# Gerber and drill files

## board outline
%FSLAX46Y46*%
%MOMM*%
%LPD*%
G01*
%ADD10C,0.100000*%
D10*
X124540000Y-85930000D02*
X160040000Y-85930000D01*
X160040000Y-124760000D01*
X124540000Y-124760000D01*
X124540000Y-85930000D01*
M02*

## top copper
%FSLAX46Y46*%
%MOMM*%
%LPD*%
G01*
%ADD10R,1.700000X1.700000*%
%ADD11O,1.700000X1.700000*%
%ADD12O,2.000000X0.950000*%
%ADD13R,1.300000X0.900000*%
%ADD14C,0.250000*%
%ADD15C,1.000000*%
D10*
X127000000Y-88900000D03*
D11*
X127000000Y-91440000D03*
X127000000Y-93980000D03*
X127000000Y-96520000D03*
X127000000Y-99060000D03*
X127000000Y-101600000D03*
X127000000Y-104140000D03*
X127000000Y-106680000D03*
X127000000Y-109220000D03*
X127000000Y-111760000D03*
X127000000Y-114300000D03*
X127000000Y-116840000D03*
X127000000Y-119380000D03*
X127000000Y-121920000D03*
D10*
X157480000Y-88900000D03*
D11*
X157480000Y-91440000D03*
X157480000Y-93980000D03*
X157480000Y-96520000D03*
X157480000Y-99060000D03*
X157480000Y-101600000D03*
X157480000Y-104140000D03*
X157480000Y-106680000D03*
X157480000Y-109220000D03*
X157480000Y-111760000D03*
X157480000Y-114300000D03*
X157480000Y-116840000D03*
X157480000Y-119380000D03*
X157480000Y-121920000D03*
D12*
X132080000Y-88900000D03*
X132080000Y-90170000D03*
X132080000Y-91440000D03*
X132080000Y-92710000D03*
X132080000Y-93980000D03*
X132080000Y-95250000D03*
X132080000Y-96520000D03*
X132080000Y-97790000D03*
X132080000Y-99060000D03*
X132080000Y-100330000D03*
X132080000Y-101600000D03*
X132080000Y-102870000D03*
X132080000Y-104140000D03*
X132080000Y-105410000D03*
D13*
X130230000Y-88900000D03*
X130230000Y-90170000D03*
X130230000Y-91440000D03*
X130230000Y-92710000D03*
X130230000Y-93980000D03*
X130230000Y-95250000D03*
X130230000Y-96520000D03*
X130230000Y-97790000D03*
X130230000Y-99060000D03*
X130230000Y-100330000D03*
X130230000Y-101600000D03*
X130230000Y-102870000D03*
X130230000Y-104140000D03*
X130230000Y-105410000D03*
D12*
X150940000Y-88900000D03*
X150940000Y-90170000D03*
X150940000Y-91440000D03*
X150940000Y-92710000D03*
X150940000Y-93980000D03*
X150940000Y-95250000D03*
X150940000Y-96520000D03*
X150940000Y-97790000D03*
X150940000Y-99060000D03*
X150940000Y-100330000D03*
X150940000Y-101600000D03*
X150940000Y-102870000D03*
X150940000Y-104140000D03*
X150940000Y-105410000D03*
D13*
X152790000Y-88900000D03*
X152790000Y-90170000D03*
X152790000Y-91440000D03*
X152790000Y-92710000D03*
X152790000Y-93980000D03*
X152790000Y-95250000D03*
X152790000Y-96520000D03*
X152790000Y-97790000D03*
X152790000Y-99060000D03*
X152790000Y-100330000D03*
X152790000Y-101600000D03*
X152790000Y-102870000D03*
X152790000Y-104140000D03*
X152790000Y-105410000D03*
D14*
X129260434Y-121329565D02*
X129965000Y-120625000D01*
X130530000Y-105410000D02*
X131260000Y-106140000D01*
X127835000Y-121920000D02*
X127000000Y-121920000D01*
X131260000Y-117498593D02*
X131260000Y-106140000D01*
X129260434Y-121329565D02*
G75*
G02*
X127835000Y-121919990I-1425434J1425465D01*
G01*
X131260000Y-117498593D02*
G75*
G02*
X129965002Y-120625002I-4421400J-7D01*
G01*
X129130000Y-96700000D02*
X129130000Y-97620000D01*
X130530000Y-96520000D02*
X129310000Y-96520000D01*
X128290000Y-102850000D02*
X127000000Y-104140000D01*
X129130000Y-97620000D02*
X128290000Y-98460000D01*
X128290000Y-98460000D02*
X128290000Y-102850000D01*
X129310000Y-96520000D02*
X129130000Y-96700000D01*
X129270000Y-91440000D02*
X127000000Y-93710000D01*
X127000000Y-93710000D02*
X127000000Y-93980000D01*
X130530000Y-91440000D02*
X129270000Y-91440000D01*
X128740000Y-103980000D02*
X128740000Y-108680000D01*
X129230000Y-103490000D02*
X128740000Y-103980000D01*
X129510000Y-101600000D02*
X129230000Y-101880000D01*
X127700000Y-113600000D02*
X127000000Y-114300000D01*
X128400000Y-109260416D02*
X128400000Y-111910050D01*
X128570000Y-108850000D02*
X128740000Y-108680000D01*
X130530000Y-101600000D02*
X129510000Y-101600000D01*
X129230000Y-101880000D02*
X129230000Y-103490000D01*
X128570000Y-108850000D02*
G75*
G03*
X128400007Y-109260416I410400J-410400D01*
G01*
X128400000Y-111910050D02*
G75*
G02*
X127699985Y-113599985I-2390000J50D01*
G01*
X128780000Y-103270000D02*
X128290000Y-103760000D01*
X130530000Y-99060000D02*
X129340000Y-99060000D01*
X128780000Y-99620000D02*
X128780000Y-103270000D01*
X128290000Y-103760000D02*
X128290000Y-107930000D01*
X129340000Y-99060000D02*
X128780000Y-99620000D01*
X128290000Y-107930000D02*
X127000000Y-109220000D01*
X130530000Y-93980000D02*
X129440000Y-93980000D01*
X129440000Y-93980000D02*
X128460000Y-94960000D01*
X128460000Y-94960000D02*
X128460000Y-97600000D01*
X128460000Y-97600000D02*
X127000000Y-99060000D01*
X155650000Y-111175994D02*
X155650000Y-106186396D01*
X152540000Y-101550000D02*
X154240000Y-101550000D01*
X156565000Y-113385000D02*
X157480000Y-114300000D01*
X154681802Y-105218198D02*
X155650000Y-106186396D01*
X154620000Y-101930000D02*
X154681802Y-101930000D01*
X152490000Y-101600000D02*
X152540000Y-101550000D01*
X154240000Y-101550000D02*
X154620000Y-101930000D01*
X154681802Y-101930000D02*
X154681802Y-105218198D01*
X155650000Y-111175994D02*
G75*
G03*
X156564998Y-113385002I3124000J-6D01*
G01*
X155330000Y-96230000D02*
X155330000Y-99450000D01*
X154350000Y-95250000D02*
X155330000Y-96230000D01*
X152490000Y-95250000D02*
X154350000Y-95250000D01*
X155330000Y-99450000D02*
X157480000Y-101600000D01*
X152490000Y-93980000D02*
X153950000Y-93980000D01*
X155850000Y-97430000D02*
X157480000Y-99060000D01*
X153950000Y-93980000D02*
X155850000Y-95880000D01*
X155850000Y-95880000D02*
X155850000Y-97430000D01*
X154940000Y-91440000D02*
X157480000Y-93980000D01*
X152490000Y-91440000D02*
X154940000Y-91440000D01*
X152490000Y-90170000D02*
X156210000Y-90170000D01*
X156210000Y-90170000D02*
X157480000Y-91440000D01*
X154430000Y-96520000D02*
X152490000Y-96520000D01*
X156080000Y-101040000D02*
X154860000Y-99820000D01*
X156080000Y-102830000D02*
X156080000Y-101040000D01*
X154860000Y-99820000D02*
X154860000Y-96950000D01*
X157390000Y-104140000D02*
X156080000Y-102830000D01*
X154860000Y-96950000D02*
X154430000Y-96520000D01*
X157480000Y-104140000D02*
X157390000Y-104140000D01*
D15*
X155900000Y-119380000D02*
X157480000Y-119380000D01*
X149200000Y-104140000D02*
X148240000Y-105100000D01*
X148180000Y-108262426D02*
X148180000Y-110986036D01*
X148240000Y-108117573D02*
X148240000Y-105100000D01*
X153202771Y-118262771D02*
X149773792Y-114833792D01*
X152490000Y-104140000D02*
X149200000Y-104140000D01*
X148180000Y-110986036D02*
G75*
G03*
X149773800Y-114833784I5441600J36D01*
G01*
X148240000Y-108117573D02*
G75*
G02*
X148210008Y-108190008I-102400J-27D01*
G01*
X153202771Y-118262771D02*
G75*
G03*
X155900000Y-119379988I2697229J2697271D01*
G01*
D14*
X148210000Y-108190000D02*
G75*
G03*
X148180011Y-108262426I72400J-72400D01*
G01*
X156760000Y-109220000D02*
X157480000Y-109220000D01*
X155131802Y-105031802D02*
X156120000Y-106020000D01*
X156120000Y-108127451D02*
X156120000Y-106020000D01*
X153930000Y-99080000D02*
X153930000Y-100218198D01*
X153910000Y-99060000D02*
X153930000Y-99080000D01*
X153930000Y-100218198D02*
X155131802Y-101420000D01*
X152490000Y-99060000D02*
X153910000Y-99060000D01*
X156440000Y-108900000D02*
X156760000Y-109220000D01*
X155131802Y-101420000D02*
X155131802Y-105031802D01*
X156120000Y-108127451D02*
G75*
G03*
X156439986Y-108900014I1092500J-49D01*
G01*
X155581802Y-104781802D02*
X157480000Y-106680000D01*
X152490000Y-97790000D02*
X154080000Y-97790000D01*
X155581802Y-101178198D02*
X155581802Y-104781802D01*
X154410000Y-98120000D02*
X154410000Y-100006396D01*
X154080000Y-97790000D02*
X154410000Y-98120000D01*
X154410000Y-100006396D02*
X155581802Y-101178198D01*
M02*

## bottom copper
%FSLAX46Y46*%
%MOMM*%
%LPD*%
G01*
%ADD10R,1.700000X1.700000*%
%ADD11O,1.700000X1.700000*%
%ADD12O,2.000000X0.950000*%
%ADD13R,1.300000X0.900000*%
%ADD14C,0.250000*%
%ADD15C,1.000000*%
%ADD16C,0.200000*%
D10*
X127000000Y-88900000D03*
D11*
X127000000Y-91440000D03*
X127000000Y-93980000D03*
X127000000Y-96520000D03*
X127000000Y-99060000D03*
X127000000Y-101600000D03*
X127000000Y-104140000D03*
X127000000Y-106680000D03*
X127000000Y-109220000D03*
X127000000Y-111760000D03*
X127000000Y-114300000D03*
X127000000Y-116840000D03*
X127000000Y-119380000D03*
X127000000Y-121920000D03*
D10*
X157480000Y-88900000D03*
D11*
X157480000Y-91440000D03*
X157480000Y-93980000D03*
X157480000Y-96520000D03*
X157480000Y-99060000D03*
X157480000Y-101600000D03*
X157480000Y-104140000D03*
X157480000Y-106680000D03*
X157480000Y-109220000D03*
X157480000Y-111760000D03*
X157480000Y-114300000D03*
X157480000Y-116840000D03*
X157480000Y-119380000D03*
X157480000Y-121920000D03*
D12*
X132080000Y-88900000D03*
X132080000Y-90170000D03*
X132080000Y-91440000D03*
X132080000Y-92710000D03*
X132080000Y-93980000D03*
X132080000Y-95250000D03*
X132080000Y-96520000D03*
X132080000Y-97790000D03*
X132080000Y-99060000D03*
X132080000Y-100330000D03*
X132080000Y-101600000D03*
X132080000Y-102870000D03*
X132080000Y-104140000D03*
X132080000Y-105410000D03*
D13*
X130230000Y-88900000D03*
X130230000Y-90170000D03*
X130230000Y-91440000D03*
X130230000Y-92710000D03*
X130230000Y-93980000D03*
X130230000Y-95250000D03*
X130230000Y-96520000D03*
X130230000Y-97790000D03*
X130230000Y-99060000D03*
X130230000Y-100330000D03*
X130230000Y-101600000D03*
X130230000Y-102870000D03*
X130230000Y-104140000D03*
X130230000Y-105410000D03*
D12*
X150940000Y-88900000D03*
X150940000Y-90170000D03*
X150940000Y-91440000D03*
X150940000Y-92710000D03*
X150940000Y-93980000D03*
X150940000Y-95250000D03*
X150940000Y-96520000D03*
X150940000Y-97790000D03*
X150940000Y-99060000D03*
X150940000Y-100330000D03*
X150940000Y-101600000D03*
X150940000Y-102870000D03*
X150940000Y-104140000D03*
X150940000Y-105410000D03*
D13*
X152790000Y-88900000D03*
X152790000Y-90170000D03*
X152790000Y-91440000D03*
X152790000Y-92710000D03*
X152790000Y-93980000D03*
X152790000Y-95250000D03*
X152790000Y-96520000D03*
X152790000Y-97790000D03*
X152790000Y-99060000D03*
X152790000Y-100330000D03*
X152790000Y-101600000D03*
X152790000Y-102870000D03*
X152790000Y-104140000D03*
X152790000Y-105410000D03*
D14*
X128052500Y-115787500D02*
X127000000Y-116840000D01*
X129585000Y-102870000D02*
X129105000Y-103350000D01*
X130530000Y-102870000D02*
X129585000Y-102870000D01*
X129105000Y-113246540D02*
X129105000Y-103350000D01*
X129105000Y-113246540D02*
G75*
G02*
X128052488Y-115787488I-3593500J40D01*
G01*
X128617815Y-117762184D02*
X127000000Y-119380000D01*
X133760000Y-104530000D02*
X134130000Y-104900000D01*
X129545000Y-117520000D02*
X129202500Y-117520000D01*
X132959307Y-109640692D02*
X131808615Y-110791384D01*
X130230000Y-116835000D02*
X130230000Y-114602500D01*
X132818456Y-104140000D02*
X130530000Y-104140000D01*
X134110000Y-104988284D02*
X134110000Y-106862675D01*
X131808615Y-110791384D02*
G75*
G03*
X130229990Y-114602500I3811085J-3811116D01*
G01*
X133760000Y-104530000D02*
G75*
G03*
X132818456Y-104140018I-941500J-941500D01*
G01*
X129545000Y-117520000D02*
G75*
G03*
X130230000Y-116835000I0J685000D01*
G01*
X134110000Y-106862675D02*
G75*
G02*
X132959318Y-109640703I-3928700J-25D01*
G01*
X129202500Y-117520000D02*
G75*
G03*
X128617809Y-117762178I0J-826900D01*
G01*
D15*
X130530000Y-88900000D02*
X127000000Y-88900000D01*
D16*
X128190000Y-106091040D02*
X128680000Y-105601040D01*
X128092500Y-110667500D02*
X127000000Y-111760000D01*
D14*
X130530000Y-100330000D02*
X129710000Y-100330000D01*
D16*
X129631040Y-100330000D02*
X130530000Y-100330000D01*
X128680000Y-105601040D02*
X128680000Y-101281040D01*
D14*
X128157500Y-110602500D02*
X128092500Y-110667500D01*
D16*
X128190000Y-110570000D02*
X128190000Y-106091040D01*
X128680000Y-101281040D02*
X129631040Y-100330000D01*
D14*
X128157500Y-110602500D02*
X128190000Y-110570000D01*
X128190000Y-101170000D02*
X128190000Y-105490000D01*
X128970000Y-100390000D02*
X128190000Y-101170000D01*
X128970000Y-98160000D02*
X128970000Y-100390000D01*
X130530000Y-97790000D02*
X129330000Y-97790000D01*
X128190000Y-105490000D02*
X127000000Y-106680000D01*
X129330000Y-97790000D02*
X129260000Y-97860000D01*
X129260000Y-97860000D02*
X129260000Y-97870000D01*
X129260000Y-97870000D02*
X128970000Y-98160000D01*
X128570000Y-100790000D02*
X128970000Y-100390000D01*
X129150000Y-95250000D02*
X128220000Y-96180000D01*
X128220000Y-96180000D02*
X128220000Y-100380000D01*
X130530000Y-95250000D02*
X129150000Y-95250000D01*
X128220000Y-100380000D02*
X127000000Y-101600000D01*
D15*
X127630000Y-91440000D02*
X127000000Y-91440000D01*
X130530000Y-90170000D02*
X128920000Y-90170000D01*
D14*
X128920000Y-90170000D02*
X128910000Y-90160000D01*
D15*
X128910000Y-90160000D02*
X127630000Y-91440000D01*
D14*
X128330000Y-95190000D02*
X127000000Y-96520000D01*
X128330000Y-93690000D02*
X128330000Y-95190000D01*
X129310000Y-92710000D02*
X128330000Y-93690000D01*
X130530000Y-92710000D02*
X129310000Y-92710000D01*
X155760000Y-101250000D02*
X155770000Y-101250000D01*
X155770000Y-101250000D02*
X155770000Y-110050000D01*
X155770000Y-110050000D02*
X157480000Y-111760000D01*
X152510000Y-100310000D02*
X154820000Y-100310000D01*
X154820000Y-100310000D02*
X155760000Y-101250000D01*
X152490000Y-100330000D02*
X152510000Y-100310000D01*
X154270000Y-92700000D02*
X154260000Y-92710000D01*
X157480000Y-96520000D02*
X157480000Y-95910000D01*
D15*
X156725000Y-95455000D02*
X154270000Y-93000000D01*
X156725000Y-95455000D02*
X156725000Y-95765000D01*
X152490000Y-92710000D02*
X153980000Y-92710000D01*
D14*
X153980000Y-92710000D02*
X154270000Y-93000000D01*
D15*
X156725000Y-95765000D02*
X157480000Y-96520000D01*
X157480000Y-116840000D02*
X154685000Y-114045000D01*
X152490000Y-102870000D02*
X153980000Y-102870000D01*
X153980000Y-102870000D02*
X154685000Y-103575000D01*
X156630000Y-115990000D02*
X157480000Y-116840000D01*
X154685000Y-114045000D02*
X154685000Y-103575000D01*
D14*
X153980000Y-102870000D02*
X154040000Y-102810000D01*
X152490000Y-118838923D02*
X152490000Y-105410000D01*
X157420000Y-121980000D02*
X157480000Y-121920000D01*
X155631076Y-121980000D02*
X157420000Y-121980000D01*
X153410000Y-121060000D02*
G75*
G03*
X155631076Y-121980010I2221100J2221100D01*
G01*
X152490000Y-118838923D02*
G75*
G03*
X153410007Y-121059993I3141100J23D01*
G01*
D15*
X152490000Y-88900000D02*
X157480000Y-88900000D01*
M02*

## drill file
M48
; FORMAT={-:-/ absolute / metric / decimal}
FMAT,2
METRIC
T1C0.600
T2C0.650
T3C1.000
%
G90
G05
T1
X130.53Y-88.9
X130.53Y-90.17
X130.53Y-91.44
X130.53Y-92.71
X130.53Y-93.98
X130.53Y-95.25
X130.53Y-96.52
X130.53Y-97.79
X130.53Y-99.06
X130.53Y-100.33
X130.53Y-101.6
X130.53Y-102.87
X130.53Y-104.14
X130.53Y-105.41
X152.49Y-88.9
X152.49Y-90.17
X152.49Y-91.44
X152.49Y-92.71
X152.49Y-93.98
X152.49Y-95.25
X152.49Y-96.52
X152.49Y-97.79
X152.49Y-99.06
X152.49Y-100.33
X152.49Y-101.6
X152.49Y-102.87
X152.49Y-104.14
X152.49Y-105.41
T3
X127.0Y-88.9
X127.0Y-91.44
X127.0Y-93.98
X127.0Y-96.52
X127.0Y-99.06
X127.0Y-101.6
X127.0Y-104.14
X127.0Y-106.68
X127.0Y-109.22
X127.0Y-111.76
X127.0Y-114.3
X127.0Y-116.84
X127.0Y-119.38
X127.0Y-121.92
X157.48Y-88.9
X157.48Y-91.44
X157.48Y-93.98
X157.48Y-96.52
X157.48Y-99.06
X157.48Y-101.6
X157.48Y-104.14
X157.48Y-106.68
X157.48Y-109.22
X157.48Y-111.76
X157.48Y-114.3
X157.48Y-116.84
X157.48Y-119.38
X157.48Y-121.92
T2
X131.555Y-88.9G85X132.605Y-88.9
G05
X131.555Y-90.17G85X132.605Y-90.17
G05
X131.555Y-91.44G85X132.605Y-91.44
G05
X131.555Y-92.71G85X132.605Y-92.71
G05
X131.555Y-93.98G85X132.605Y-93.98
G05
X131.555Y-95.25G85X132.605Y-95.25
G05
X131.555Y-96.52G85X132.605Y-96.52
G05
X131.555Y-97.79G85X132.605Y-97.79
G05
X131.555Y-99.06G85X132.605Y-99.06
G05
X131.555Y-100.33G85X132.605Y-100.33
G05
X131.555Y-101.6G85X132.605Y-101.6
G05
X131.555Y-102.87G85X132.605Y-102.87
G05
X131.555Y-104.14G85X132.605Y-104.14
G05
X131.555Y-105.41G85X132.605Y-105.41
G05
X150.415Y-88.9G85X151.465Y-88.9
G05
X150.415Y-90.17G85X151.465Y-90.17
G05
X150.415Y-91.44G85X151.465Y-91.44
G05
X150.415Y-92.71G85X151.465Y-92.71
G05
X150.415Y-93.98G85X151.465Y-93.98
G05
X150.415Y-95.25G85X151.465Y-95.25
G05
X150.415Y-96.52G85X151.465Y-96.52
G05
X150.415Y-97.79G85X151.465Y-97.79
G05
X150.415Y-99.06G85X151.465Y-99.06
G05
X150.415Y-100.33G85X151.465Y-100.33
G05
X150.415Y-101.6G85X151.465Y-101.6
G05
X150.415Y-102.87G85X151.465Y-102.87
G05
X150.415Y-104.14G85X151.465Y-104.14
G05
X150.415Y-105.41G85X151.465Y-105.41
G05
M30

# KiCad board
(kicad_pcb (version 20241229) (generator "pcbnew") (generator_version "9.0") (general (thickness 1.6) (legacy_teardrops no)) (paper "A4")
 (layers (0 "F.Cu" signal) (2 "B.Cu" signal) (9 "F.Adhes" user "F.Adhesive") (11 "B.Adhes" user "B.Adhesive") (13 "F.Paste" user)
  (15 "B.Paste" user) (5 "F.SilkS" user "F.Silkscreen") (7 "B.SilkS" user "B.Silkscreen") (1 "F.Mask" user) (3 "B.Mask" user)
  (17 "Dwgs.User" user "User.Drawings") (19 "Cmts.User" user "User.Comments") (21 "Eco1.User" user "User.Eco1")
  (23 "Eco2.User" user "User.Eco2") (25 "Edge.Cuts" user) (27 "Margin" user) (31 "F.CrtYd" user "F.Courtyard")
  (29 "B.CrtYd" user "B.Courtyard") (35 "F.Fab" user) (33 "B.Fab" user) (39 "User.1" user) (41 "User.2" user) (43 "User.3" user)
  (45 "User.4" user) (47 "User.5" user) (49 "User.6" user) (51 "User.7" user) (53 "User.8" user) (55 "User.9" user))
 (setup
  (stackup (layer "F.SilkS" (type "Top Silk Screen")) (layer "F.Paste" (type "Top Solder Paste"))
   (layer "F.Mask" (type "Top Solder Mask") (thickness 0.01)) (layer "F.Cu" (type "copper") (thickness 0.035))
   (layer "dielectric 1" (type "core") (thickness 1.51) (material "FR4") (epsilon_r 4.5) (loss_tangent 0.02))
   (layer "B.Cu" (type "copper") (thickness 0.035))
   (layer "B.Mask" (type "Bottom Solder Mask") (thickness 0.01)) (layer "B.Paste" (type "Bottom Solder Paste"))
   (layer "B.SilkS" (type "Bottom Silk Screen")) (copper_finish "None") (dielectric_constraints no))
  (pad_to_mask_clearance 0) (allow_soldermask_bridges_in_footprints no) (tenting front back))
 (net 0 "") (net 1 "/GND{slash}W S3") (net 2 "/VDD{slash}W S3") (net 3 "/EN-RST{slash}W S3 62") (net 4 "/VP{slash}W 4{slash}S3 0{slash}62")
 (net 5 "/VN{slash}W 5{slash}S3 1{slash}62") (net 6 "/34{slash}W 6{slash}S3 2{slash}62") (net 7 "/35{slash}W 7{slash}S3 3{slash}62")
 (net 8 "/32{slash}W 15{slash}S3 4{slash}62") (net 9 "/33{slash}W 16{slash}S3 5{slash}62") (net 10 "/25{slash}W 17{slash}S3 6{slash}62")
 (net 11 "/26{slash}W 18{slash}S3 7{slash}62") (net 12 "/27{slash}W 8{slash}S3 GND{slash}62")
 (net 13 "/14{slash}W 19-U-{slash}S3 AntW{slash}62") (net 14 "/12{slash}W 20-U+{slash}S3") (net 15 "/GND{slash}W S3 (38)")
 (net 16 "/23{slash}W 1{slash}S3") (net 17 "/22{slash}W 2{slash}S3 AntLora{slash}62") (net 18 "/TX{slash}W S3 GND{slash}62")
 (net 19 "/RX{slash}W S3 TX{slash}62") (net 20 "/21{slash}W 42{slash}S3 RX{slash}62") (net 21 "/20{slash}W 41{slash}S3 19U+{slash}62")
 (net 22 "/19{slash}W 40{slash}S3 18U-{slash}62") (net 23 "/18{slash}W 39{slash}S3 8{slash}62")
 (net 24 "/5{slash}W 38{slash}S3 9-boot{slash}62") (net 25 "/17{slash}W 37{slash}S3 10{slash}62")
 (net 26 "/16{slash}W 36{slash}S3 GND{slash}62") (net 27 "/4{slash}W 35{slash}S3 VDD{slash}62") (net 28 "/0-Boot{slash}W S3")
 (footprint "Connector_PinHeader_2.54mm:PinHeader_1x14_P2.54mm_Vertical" (layer "F.Cu") (at 127 88.9)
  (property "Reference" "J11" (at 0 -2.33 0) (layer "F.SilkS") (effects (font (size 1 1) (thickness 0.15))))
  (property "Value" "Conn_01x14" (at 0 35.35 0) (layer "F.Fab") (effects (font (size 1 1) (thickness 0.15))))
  (pad "1" thru_hole rect (at 0 0) (size 1.7 1.7) (drill 1) (layers "*.Cu" "*.Mask") (remove_unused_layers no) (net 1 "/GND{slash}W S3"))
  (pad "2" thru_hole oval (at 0 2.54) (size 1.7 1.7) (drill 1) (layers "*.Cu" "*.Mask") (remove_unused_layers no) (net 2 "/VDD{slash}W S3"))
  (pad "3" thru_hole oval (at 0 5.08) (size 1.7 1.7) (drill 1) (layers "*.Cu" "*.Mask") (remove_unused_layers no)
   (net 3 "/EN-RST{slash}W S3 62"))
  (pad "4" thru_hole oval (at 0 7.62) (size 1.7 1.7) (drill 1) (layers "*.Cu" "*.Mask") (remove_unused_layers no)
   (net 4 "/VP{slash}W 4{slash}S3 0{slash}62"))
  (pad "5" thru_hole oval (at 0 10.16) (size 1.7 1.7) (drill 1) (layers "*.Cu" "*.Mask") (remove_unused_layers no)
   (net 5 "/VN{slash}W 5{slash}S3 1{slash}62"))
  (pad "6" thru_hole oval (at 0 12.7) (size 1.7 1.7) (drill 1) (layers "*.Cu" "*.Mask") (remove_unused_layers no)
   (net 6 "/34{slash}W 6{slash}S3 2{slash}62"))
  (pad "7" thru_hole oval (at 0 15.24) (size 1.7 1.7) (drill 1) (layers "*.Cu" "*.Mask") (remove_unused_layers no)
   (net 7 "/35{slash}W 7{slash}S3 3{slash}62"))
  (pad "8" thru_hole oval (at 0 17.78) (size 1.7 1.7) (drill 1) (layers "*.Cu" "*.Mask") (remove_unused_layers no)
   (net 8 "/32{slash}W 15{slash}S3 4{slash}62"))
  (pad "9" thru_hole oval (at 0 20.32) (size 1.7 1.7) (drill 1) (layers "*.Cu" "*.Mask") (remove_unused_layers no)
   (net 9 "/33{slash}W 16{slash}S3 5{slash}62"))
  (pad "10" thru_hole oval (at 0 22.86) (size 1.7 1.7) (drill 1) (layers "*.Cu" "*.Mask") (remove_unused_layers no)
   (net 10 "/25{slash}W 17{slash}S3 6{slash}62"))
  (pad "11" thru_hole oval (at 0 25.4) (size 1.7 1.7) (drill 1) (layers "*.Cu" "*.Mask") (remove_unused_layers no)
   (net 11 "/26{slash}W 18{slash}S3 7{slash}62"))
  (pad "12" thru_hole oval (at 0 27.94) (size 1.7 1.7) (drill 1) (layers "*.Cu" "*.Mask") (remove_unused_layers no)
   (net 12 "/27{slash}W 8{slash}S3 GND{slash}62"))
  (pad "13" thru_hole oval (at 0 30.48) (size 1.7 1.7) (drill 1) (layers "*.Cu" "*.Mask") (remove_unused_layers no)
   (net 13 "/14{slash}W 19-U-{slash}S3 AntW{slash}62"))
  (pad "14" thru_hole oval (at 0 33.02) (size 1.7 1.7) (drill 1) (layers "*.Cu" "*.Mask") (remove_unused_layers no)
   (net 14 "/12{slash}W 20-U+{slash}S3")))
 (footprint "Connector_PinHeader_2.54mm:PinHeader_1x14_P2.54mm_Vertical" (layer "F.Cu") (at 157.48 88.9)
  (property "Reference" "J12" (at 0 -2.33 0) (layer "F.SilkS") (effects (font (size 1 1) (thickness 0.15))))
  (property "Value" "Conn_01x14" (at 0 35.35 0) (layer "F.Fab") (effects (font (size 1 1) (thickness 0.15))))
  (pad "1" thru_hole rect (at 0 0) (size 1.7 1.7) (drill 1) (layers "*.Cu" "*.Mask") (remove_unused_layers no)
   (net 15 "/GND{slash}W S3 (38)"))
  (pad "2" thru_hole oval (at 0 2.54) (size 1.7 1.7) (drill 1) (layers "*.Cu" "*.Mask") (remove_unused_layers no)
   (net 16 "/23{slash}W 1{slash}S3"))
  (pad "3" thru_hole oval (at 0 5.08) (size 1.7 1.7) (drill 1) (layers "*.Cu" "*.Mask") (remove_unused_layers no)
   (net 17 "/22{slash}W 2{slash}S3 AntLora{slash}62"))
  (pad "4" thru_hole oval (at 0 7.62) (size 1.7 1.7) (drill 1) (layers "*.Cu" "*.Mask") (remove_unused_layers no)
   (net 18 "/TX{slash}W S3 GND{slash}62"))
  (pad "5" thru_hole oval (at 0 10.16) (size 1.7 1.7) (drill 1) (layers "*.Cu" "*.Mask") (remove_unused_layers no)
   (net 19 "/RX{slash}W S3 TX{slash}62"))
  (pad "6" thru_hole oval (at 0 12.7) (size 1.7 1.7) (drill 1) (layers "*.Cu" "*.Mask") (remove_unused_layers no)
   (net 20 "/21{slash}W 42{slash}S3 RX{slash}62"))
  (pad "7" thru_hole oval (at 0 15.24) (size 1.7 1.7) (drill 1) (layers "*.Cu" "*.Mask") (remove_unused_layers no)
   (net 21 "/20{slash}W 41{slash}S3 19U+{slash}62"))
  (pad "8" thru_hole oval (at 0 17.78) (size 1.7 1.7) (drill 1) (layers "*.Cu" "*.Mask") (remove_unused_layers no)
   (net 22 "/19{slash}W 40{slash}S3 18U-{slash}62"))
  (pad "9" thru_hole oval (at 0 20.32) (size 1.7 1.7) (drill 1) (layers "*.Cu" "*.Mask") (remove_unused_layers no)
   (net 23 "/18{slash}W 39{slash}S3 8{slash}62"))
  (pad "10" thru_hole oval (at 0 22.86) (size 1.7 1.7) (drill 1) (layers "*.Cu" "*.Mask") (remove_unused_layers no)
   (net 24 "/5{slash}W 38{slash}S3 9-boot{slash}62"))
  (pad "11" thru_hole oval (at 0 25.4) (size 1.7 1.7) (drill 1) (layers "*.Cu" "*.Mask") (remove_unused_layers no)
   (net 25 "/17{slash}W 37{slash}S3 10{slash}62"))
  (pad "12" thru_hole oval (at 0 27.94) (size 1.7 1.7) (drill 1) (layers "*.Cu" "*.Mask") (remove_unused_layers no)
   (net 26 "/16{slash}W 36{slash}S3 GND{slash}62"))
  (pad "13" thru_hole oval (at 0 30.48) (size 1.7 1.7) (drill 1) (layers "*.Cu" "*.Mask") (remove_unused_layers no)
   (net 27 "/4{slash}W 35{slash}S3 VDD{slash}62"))
  (pad "14" thru_hole oval (at 0 33.02) (size 1.7 1.7) (drill 1) (layers "*.Cu" "*.Mask") (remove_unused_layers no)
   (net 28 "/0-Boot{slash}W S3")))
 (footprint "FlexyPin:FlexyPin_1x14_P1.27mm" (layer "F.Cu") (at 130.53 88.9)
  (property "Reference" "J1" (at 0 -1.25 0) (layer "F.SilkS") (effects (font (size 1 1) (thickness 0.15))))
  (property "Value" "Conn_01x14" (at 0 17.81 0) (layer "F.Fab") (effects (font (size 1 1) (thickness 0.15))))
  (pad "" thru_hole oval (at 1.55 0) (size 2 0.95) (drill oval 1.7 0.65) (layers "*.Cu" "*.Mask") (remove_unused_layers no))
  (pad "" thru_hole oval (at 1.55 1.27) (size 2 0.95) (drill oval 1.7 0.65) (layers "*.Cu" "*.Mask") (remove_unused_layers no))
  (pad "" thru_hole oval (at 1.55 2.54) (size 2 0.95) (drill oval 1.7 0.65) (layers "*.Cu" "*.Mask") (remove_unused_layers no))
  (pad "" thru_hole oval (at 1.55 3.81) (size 2 0.95) (drill oval 1.7 0.65) (layers "*.Cu" "*.Mask") (remove_unused_layers no))
  (pad "" thru_hole oval (at 1.55 5.08) (size 2 0.95) (drill oval 1.7 0.65) (layers "*.Cu" "*.Mask") (remove_unused_layers no))
  (pad "" thru_hole oval (at 1.55 6.35) (size 2 0.95) (drill oval 1.7 0.65) (layers "*.Cu" "*.Mask") (remove_unused_layers no))
  (pad "" thru_hole oval (at 1.55 7.62) (size 2 0.95) (drill oval 1.7 0.65) (layers "*.Cu" "*.Mask") (remove_unused_layers no))
  (pad "" thru_hole oval (at 1.55 8.89) (size 2 0.95) (drill oval 1.7 0.65) (layers "*.Cu" "*.Mask") (remove_unused_layers no))
  (pad "" thru_hole oval (at 1.55 10.16) (size 2 0.95) (drill oval 1.7 0.65) (layers "*.Cu" "*.Mask") (remove_unused_layers no))
  (pad "" thru_hole oval (at 1.55 11.43) (size 2 0.95) (drill oval 1.7 0.65) (layers "*.Cu" "*.Mask") (remove_unused_layers no))
  (pad "" thru_hole oval (at 1.55 12.7) (size 2 0.95) (drill oval 1.7 0.65) (layers "*.Cu" "*.Mask") (remove_unused_layers no))
  (pad "" thru_hole oval (at 1.55 13.97) (size 2 0.95) (drill oval 1.7 0.65) (layers "*.Cu" "*.Mask") (remove_unused_layers no))
  (pad "" thru_hole oval (at 1.55 15.24) (size 2 0.95) (drill oval 1.7 0.65) (layers "*.Cu" "*.Mask") (remove_unused_layers no))
  (pad "" thru_hole oval (at 1.55 16.51) (size 2 0.95) (drill oval 1.7 0.65) (layers "*.Cu" "*.Mask") (remove_unused_layers no))
  (pad "1" thru_hole rect (at 0 0) (size 1.3 0.9) (drill 0.6 (offset -0.3 0)) (layers "*.Cu" "*.Mask") (remove_unused_layers no)
   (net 1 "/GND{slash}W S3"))
  (pad "2" thru_hole rect (at 0 1.27) (size 1.3 0.9) (drill 0.6 (offset -0.3 0)) (layers "*.Cu" "*.Mask") (remove_unused_layers no)
   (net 2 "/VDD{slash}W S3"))
  (pad "3" thru_hole rect (at 0 2.54) (size 1.3 0.9) (drill 0.6 (offset -0.3 0)) (layers "*.Cu" "*.Mask") (remove_unused_layers no)
   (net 3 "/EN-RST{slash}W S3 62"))
  (pad "4" thru_hole rect (at 0 3.81) (size 1.3 0.9) (drill 0.6 (offset -0.3 0)) (layers "*.Cu" "*.Mask") (remove_unused_layers no)
   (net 4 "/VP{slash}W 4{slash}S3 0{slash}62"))
  (pad "5" thru_hole rect (at 0 5.08) (size 1.3 0.9) (drill 0.6 (offset -0.3 0)) (layers "*.Cu" "*.Mask") (remove_unused_layers no)
   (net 5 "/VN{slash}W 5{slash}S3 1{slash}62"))
  (pad "6" thru_hole rect (at 0 6.35) (size 1.3 0.9) (drill 0.6 (offset -0.3 0)) (layers "*.Cu" "*.Mask") (remove_unused_layers no)
   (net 6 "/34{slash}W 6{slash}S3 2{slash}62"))
  (pad "7" thru_hole rect (at 0 7.62) (size 1.3 0.9) (drill 0.6 (offset -0.3 0)) (layers "*.Cu" "*.Mask") (remove_unused_layers no)
   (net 7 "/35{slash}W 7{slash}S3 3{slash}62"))
  (pad "8" thru_hole rect (at 0 8.89) (size 1.3 0.9) (drill 0.6 (offset -0.3 0)) (layers "*.Cu" "*.Mask") (remove_unused_layers no)
   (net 8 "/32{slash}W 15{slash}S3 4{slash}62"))
  (pad "9" thru_hole rect (at 0 10.16) (size 1.3 0.9) (drill 0.6 (offset -0.3 0)) (layers "*.Cu" "*.Mask") (remove_unused_layers no)
   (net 9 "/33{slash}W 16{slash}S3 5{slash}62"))
  (pad "10" thru_hole rect (at 0 11.43) (size 1.3 0.9) (drill 0.6 (offset -0.3 0)) (layers "*.Cu" "*.Mask") (remove_unused_layers no)
   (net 10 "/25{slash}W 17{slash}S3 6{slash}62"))
  (pad "11" thru_hole rect (at 0 12.7) (size 1.3 0.9) (drill 0.6 (offset -0.3 0)) (layers "*.Cu" "*.Mask") (remove_unused_layers no)
   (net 11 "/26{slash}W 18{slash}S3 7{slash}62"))
  (pad "12" thru_hole rect (at 0 13.97) (size 1.3 0.9) (drill 0.6 (offset -0.3 0)) (layers "*.Cu" "*.Mask") (remove_unused_layers no)
   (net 12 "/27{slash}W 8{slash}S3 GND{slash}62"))
  (pad "13" thru_hole rect (at 0 15.24) (size 1.3 0.9) (drill 0.6 (offset -0.3 0)) (layers "*.Cu" "*.Mask") (remove_unused_layers no)
   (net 13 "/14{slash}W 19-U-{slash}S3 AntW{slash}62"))
  (pad "14" thru_hole rect (at 0 16.51) (size 1.3 0.9) (drill 0.6 (offset -0.3 0)) (layers "*.Cu" "*.Mask") (remove_unused_layers no)
   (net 14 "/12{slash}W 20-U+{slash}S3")))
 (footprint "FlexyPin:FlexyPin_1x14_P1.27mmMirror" (layer "F.Cu") (at 152.49 88.9)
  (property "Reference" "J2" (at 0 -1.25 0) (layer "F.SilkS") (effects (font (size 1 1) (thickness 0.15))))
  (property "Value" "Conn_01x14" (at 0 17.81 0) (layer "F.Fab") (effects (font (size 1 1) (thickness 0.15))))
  (pad "" thru_hole oval (at -1.55 0) (size 2 0.95) (drill oval 1.7 0.65) (layers "*.Cu" "*.Mask") (remove_unused_layers no))
  (pad "" thru_hole oval (at -1.55 1.27) (size 2 0.95) (drill oval 1.7 0.65) (layers "*.Cu" "*.Mask") (remove_unused_layers no))
  (pad "" thru_hole oval (at -1.55 2.54) (size 2 0.95) (drill oval 1.7 0.65) (layers "*.Cu" "*.Mask") (remove_unused_layers no))
  (pad "" thru_hole oval (at -1.55 3.81) (size 2 0.95) (drill oval 1.7 0.65) (layers "*.Cu" "*.Mask") (remove_unused_layers no))
  (pad "" thru_hole oval (at -1.55 5.08) (size 2 0.95) (drill oval 1.7 0.65) (layers "*.Cu" "*.Mask") (remove_unused_layers no))
  (pad "" thru_hole oval (at -1.55 6.35) (size 2 0.95) (drill oval 1.7 0.65) (layers "*.Cu" "*.Mask") (remove_unused_layers no))
  (pad "" thru_hole oval (at -1.55 7.62) (size 2 0.95) (drill oval 1.7 0.65) (layers "*.Cu" "*.Mask") (remove_unused_layers no))
  (pad "" thru_hole oval (at -1.55 8.89) (size 2 0.95) (drill oval 1.7 0.65) (layers "*.Cu" "*.Mask") (remove_unused_layers no))
  (pad "" thru_hole oval (at -1.55 10.16) (size 2 0.95) (drill oval 1.7 0.65) (layers "*.Cu" "*.Mask") (remove_unused_layers no))
  (pad "" thru_hole oval (at -1.55 11.43) (size 2 0.95) (drill oval 1.7 0.65) (layers "*.Cu" "*.Mask") (remove_unused_layers no))
  (pad "" thru_hole oval (at -1.55 12.7) (size 2 0.95) (drill oval 1.7 0.65) (layers "*.Cu" "*.Mask") (remove_unused_layers no))
  (pad "" thru_hole oval (at -1.55 13.97) (size 2 0.95) (drill oval 1.7 0.65) (layers "*.Cu" "*.Mask") (remove_unused_layers no))
  (pad "" thru_hole oval (at -1.55 15.24) (size 2 0.95) (drill oval 1.7 0.65) (layers "*.Cu" "*.Mask") (remove_unused_layers no))
  (pad "" thru_hole oval (at -1.55 16.51) (size 2 0.95) (drill oval 1.7 0.65) (layers "*.Cu" "*.Mask") (remove_unused_layers no))
  (pad "1" thru_hole rect (at 0 0) (size 1.3 0.9) (drill 0.6 (offset 0.3 0)) (layers "*.Cu" "*.Mask") (remove_unused_layers no)
   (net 15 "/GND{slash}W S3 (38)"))
  (pad "2" thru_hole rect (at 0 1.27) (size 1.3 0.9) (drill 0.6 (offset 0.3 0)) (layers "*.Cu" "*.Mask") (remove_unused_layers no)
   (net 16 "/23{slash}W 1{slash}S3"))
  (pad "3" thru_hole rect (at 0 2.54) (size 1.3 0.9) (drill 0.6 (offset 0.3 0)) (layers "*.Cu" "*.Mask") (remove_unused_layers no)
   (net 17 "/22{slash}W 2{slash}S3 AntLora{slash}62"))
  (pad "4" thru_hole rect (at 0 3.81) (size 1.3 0.9) (drill 0.6 (offset 0.3 0)) (layers "*.Cu" "*.Mask") (remove_unused_layers no)
   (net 18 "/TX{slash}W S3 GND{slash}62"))
  (pad "5" thru_hole rect (at 0 5.08) (size 1.3 0.9) (drill 0.6 (offset 0.3 0)) (layers "*.Cu" "*.Mask") (remove_unused_layers no)
   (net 19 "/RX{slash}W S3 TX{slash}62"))
  (pad "6" thru_hole rect (at 0 6.35) (size 1.3 0.9) (drill 0.6 (offset 0.3 0)) (layers "*.Cu" "*.Mask") (remove_unused_layers no)
   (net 20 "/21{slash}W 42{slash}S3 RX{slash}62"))
  (pad "7" thru_hole rect (at 0 7.62) (size 1.3 0.9) (drill 0.6 (offset 0.3 0)) (layers "*.Cu" "*.Mask") (remove_unused_layers no)
   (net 21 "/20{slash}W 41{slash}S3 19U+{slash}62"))
  (pad "8" thru_hole rect (at 0 8.89) (size 1.3 0.9) (drill 0.6 (offset 0.3 0)) (layers "*.Cu" "*.Mask") (remove_unused_layers no)
   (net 22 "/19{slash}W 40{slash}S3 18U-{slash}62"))
  (pad "9" thru_hole rect (at 0 10.16) (size 1.3 0.9) (drill 0.6 (offset 0.3 0)) (layers "*.Cu" "*.Mask") (remove_unused_layers no)
   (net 23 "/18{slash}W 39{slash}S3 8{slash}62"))
  (pad "10" thru_hole rect (at 0 11.43) (size 1.3 0.9) (drill 0.6 (offset 0.3 0)) (layers "*.Cu" "*.Mask") (remove_unused_layers no)
   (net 24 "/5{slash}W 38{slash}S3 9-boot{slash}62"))
  (pad "11" thru_hole rect (at 0 12.7) (size 1.3 0.9) (drill 0.6 (offset 0.3 0)) (layers "*.Cu" "*.Mask") (remove_unused_layers no)
   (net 25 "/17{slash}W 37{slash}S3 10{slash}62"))
  (pad "12" thru_hole rect (at 0 13.97) (size 1.3 0.9) (drill 0.6 (offset 0.3 0)) (layers "*.Cu" "*.Mask") (remove_unused_layers no)
   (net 26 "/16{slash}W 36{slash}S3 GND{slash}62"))
  (pad "13" thru_hole rect (at 0 15.24) (size 1.3 0.9) (drill 0.6 (offset 0.3 0)) (layers "*.Cu" "*.Mask") (remove_unused_layers no)
   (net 27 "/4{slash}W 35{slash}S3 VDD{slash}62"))
  (pad "14" thru_hole rect (at 0 16.51) (size 1.3 0.9) (drill 0.6 (offset 0.3 0)) (layers "*.Cu" "*.Mask") (remove_unused_layers no)
   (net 28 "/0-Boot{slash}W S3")))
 (gr_rect (start 124.54 85.93) (end 160.04 124.76) (stroke (width 0.1) (type default)) (fill no) (layer "Edge.Cuts"))
 (segment (start 128.0525 115.7875) (end 127 116.84) (width 0.25) (layer "B.Cu") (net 12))
 (segment (start 129.585 102.87) (end 129.105 103.35) (width 0.25) (layer "B.Cu") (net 12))
 (segment (start 130.53 102.87) (end 129.585 102.87) (width 0.25) (layer "B.Cu") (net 12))
 (segment (start 129.105 113.24654) (end 129.105 103.35) (width 0.25) (layer "B.Cu") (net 12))
 (arc (start 129.105 113.24654) (mid 128.831464 114.621697) (end 128.0525 115.7875) (width 0.25) (layer "B.Cu") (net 12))
 (segment (start 129.260434 121.329565) (end 129.965 120.625) (width 0.25) (layer "F.Cu") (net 14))
 (segment (start 130.53 105.41) (end 131.26 106.14) (width 0.25) (layer "F.Cu") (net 14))
 (segment (start 127.835 121.92) (end 127 121.92) (width 0.25) (layer "F.Cu") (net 14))
 (segment (start 131.26 117.498593) (end 131.26 106.14) (width 0.25) (layer "F.Cu") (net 14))
 (arc (start 129.260434 121.329565) (mid 128.606439 121.76655) (end 127.835 121.92) (width 0.25) (layer "F.Cu") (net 14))
 (arc (start 131.26 117.498593) (mid 130.92344 119.190592) (end 129.965 120.625) (width 0.25) (layer "F.Cu") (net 14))
 (segment (start 128.617815 117.762184) (end 127 119.38) (width 0.25) (layer "B.Cu") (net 13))
 (segment (start 133.76 104.53) (end 134.13 104.9) (width 0.25) (layer "B.Cu") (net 13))
 (segment (start 129.545 117.52) (end 129.2025 117.52) (width 0.25) (layer "B.Cu") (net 13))
 (segment (start 132.959307 109.640692) (end 131.808615 110.791384) (width 0.25) (layer "B.Cu") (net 13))
 (segment (start 130.23 116.835) (end 130.23 114.6025) (width 0.25) (layer "B.Cu") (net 13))
 (segment (start 132.818456 104.14) (end 130.53 104.14) (width 0.25) (layer "B.Cu") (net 13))
 (segment (start 134.11 104.988284) (end 134.11 106.862675) (width 0.25) (layer "B.Cu") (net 13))
 (arc (start 131.808615 110.791384) (mid 130.640268 112.539938) (end 130.23 114.6025) (width 0.25) (layer "B.Cu") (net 13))
 (arc (start 133.76 104.53) (mid 133.328016 104.241357) (end 132.818456 104.14) (width 0.25) (layer "B.Cu") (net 13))
 (arc (start 129.545 117.52) (mid 130.029368 117.319368) (end 130.23 116.835) (width 0.25) (layer "B.Cu") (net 13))
 (arc (start 134.11 106.862675) (mid 133.810944 108.366127) (end 132.959307 109.640692) (width 0.25) (layer "B.Cu") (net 13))
 (arc (start 129.2025 117.52) (mid 128.886071 117.582941) (end 128.617815 117.762184) (width 0.25) (layer "B.Cu") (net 13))
 (segment (start 130.53 88.9) (end 127 88.9) (width 1) (layer "B.Cu") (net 1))
 (segment (start 129.13 96.7) (end 129.13 97.62) (width 0.25) (layer "F.Cu") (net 7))
 (segment (start 130.53 96.52) (end 129.31 96.52) (width 0.25) (layer "F.Cu") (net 7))
 (segment (start 128.29 102.85) (end 127 104.14) (width 0.25) (layer "F.Cu") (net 7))
 (segment (start 129.13 97.62) (end 128.29 98.46) (width 0.25) (layer "F.Cu") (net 7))
 (segment (start 128.29 98.46) (end 128.29 102.85) (width 0.25) (layer "F.Cu") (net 7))
 (segment (start 129.31 96.52) (end 129.13 96.7) (width 0.25) (layer "F.Cu") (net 7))
 (segment (start 128.19 106.09104) (end 128.68 105.60104) (width 0.2) (layer "B.Cu") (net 10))
 (segment (start 128.0925 110.6675) (end 127 111.76) (width 0.2) (layer "B.Cu") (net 10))
 (segment (start 130.53 100.33) (end 129.71 100.33) (width 0.25) (layer "B.Cu") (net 10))
 (segment (start 129.63104 100.33) (end 130.53 100.33) (width 0.2) (layer "B.Cu") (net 10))
 (segment (start 128.68 105.60104) (end 128.68 101.28104) (width 0.2) (layer "B.Cu") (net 10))
 (segment (start 128.1575 110.6025) (end 128.0925 110.6675) (width 0.25) (layer "B.Cu") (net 10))
 (segment (start 128.19 110.57) (end 128.19 106.09104) (width 0.2) (layer "B.Cu") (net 10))
 (segment (start 128.68 101.28104) (end 129.63104 100.33) (width 0.2) (layer "B.Cu") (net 10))
 (segment (start 128.1575 110.6025) (end 128.19 110.57) (width 0.25) (layer "B.Cu") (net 10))
 (segment (start 128.19 101.17) (end 128.19 105.49) (width 0.25) (layer "B.Cu") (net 8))
 (segment (start 128.97 100.39) (end 128.19 101.17) (width 0.25) (layer "B.Cu") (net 8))
 (segment (start 128.97 98.16) (end 128.97 100.39) (width 0.25) (layer "B.Cu") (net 8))
 (segment (start 130.53 97.79) (end 129.33 97.79) (width 0.25) (layer "B.Cu") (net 8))
 (segment (start 128.19 105.49) (end 127 106.68) (width 0.25) (layer "B.Cu") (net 8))
 (segment (start 129.33 97.79) (end 129.26 97.86) (width 0.25) (layer "B.Cu") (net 8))
 (segment (start 129.26 97.86) (end 129.26 97.87) (width 0.25) (layer "B.Cu") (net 8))
 (segment (start 129.26 97.87) (end 128.97 98.16) (width 0.25) (layer "B.Cu") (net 8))
 (segment (start 128.57 100.79) (end 128.97 100.39) (width 0.25) (layer "B.Cu") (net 8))
 (segment (start 129.27 91.44) (end 127 93.71) (width 0.25) (layer "F.Cu") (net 3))
 (segment (start 127 93.71) (end 127 93.98) (width 0.25) (layer "F.Cu") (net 3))
 (segment (start 130.53 91.44) (end 129.27 91.44) (width 0.25) (layer "F.Cu") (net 3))
 (segment (start 128.74 103.98) (end 128.74 108.68) (width 0.25) (layer "F.Cu") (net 11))
 (segment (start 129.23 103.49) (end 128.74 103.98) (width 0.25) (layer "F.Cu") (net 11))
 (segment (start 129.51 101.6) (end 129.23 101.88) (width 0.25) (layer "F.Cu") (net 11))
 (segment (start 127.7 113.6) (end 127 114.3) (width 0.25) (layer "F.Cu") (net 11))
 (segment (start 128.4 109.260416) (end 128.4 111.91005) (width 0.25) (layer "F.Cu") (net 11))
 (segment (start 128.57 108.85) (end 128.74 108.68) (width 0.25) (layer "F.Cu") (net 11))
 (segment (start 130.53 101.6) (end 129.51 101.6) (width 0.25) (layer "F.Cu") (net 11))
 (segment (start 129.23 101.88) (end 129.23 103.49) (width 0.25) (layer "F.Cu") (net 11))
 (arc (start 128.57 108.85) (mid 128.444181 109.0383) (end 128.4 109.260416) (width 0.25) (layer "F.Cu") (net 11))
 (arc (start 128.4 111.91005) (mid 128.218075 112.824644) (end 127.7 113.6) (width 0.25) (layer "F.Cu") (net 11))
 (segment (start 129.15 95.25) (end 128.22 96.18) (width 0.25) (layer "B.Cu") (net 6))
 (segment (start 128.22 96.18) (end 128.22 100.38) (width 0.25) (layer "B.Cu") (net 6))
 (segment (start 130.53 95.25) (end 129.15 95.25) (width 0.25) (layer "B.Cu") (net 6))
 (segment (start 128.22 100.38) (end 127 101.6) (width 0.25) (layer "B.Cu") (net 6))
 (segment (start 127.63 91.44) (end 127 91.44) (width 1) (layer "B.Cu") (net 2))
 (segment (start 130.53 90.17) (end 128.92 90.17) (width 1) (layer "B.Cu") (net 2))
 (segment (start 128.92 90.17) (end 128.91 90.16) (width 0.25) (layer "B.Cu") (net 2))
 (segment (start 128.91 90.16) (end 127.63 91.44) (width 1) (layer "B.Cu") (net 2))
 (segment (start 128.33 95.19) (end 127 96.52) (width 0.25) (layer "B.Cu") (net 4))
 (segment (start 128.33 93.69) (end 128.33 95.19) (width 0.25) (layer "B.Cu") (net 4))
 (segment (start 129.31 92.71) (end 128.33 93.69) (width 0.25) (layer "B.Cu") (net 4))
 (segment (start 130.53 92.71) (end 129.31 92.71) (width 0.25) (layer "B.Cu") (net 4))
 (segment (start 128.78 103.27) (end 128.29 103.76) (width 0.25) (layer "F.Cu") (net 9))
 (segment (start 130.53 99.06) (end 129.34 99.06) (width 0.25) (layer "F.Cu") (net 9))
 (segment (start 128.78 99.62) (end 128.78 103.27) (width 0.25) (layer "F.Cu") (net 9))
 (segment (start 128.29 103.76) (end 128.29 107.93) (width 0.25) (layer "F.Cu") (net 9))
 (segment (start 129.34 99.06) (end 128.78 99.62) (width 0.25) (layer "F.Cu") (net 9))
 (segment (start 128.29 107.93) (end 127 109.22) (width 0.25) (layer "F.Cu") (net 9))
 (segment (start 130.53 93.98) (end 129.44 93.98) (width 0.25) (layer "F.Cu") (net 5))
 (segment (start 129.44 93.98) (end 128.46 94.96) (width 0.25) (layer "F.Cu") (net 5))
 (segment (start 128.46 94.96) (end 128.46 97.6) (width 0.25) (layer "F.Cu") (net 5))
 (segment (start 128.46 97.6) (end 127 99.06) (width 0.25) (layer "F.Cu") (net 5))
 (segment (start 155.76 101.25) (end 155.77 101.25) (width 0.25) (layer "B.Cu") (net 24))
 (segment (start 155.77 101.25) (end 155.77 110.05) (width 0.25) (layer "B.Cu") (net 24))
 (segment (start 155.77 110.05) (end 157.48 111.76) (width 0.25) (layer "B.Cu") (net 24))
 (segment (start 152.51 100.31) (end 154.82 100.31) (width 0.25) (layer "B.Cu") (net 24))
 (segment (start 154.82 100.31) (end 155.76 101.25) (width 0.25) (layer "B.Cu") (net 24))
 (segment (start 152.49 100.33) (end 152.51 100.31) (width 0.25) (layer "B.Cu") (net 24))
 (segment (start 155.65 111.175994) (end 155.65 106.186396) (width 0.25) (layer "F.Cu") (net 25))
 (segment (start 152.54 101.55) (end 154.24 101.55) (width 0.25) (layer "F.Cu") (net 25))
 (segment (start 156.565 113.385) (end 157.48 114.3) (width 0.25) (layer "F.Cu") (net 25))
 (segment (start 154.681802 105.218198) (end 155.65 106.186396) (width 0.25) (layer "F.Cu") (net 25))
 (segment (start 154.62 101.93) (end 154.681802 101.93) (width 0.25) (layer "F.Cu") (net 25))
 (segment (start 152.49 101.6) (end 152.54 101.55) (width 0.25) (layer "F.Cu") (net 25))
 (segment (start 154.24 101.55) (end 154.62 101.93) (width 0.25) (layer "F.Cu") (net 25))
 (segment (start 154.681802 101.93) (end 154.681802 105.218198) (width 0.25) (layer "F.Cu") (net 25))
 (arc (start 155.65 111.175994) (mid 155.8878 112.371499) (end 156.565 113.385) (width 0.25) (layer "F.Cu") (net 25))
 (segment (start 155.33 96.23) (end 155.33 99.45) (width 0.25) (layer "F.Cu") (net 20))
 (segment (start 154.35 95.25) (end 155.33 96.23) (width 0.25) (layer "F.Cu") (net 20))
 (segment (start 152.49 95.25) (end 154.35 95.25) (width 0.25) (layer "F.Cu") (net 20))
 (segment (start 155.33 99.45) (end 157.48 101.6) (width 0.25) (layer "F.Cu") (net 20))
 (segment (start 154.27 92.7) (end 154.26 92.71) (width 0.25) (layer "B.Cu") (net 18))
 (segment (start 157.48 96.52) (end 157.48 95.91) (width 0.25) (layer "B.Cu") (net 18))
 (segment (start 156.725 95.455) (end 154.27 93) (width 1) (layer "B.Cu") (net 18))
 (segment (start 156.725 95.455) (end 156.725 95.765) (width 1) (layer "B.Cu") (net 18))
 (segment (start 152.49 92.71) (end 153.98 92.71) (width 1) (layer "B.Cu") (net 18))
 (segment (start 153.98 92.71) (end 154.27 93) (width 0.25) (layer "B.Cu") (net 18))
 (segment (start 156.725 95.765) (end 157.48 96.52) (width 1) (layer "B.Cu") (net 18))
 (segment (start 152.49 93.98) (end 153.95 93.98) (width 0.25) (layer "F.Cu") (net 19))
 (segment (start 155.85 97.43) (end 157.48 99.06) (width 0.25) (layer "F.Cu") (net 19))
 (segment (start 153.95 93.98) (end 155.85 95.88) (width 0.25) (layer "F.Cu") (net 19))
 (segment (start 155.85 95.88) (end 155.85 97.43) (width 0.25) (layer "F.Cu") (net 19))
 (segment (start 154.94 91.44) (end 157.48 93.98) (width 0.25) (layer "F.Cu") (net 17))
 (segment (start 152.49 91.44) (end 154.94 91.44) (width 0.25) (layer "F.Cu") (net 17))
 (segment (start 157.48 116.84) (end 154.685 114.045) (width 1) (layer "B.Cu") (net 26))
 (segment (start 152.49 102.87) (end 153.98 102.87) (width 1) (layer "B.Cu") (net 26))
 (segment (start 153.98 102.87) (end 154.685 103.575) (width 1) (layer "B.Cu") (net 26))
 (segment (start 156.63 115.99) (end 157.48 116.84) (width 1) (layer "B.Cu") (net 26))
 (segment (start 154.685 114.045) (end 154.685 103.575) (width 1) (layer "B.Cu") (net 26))
 (segment (start 153.98 102.87) (end 154.04 102.81) (width 0.25) (layer "B.Cu") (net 26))
 (segment (start 152.49 118.838923) (end 152.49 105.41) (width 0.25) (layer "B.Cu") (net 28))
 (segment (start 157.42 121.98) (end 157.48 121.92) (width 0.25) (layer "B.Cu") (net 28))
 (segment (start 155.631076 121.98) (end 157.42 121.98) (width 0.25) (layer "B.Cu") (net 28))
 (arc (start 153.41 121.06) (mid 154.429038 121.740899) (end 155.631076 121.98) (width 0.25) (layer "B.Cu") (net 28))
 (arc (start 152.49 118.838923) (mid 152.7291 120.040961) (end 153.41 121.06) (width 0.25) (layer "B.Cu") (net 28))
 (segment (start 152.49 90.17) (end 156.21 90.17) (width 0.25) (layer "F.Cu") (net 16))
 (segment (start 156.21 90.17) (end 157.48 91.44) (width 0.25) (layer "F.Cu") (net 16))
 (segment (start 152.49 88.9) (end 157.48 88.9) (width 1) (layer "B.Cu") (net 15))
 (segment (start 154.43 96.52) (end 152.49 96.52) (width 0.25) (layer "F.Cu") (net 21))
 (segment (start 156.08 101.04) (end 154.86 99.82) (width 0.25) (layer "F.Cu") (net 21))
 (segment (start 156.08 102.83) (end 156.08 101.04) (width 0.25) (layer "F.Cu") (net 21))
 (segment (start 154.86 99.82) (end 154.86 96.95) (width 0.25) (layer "F.Cu") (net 21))
 (segment (start 157.39 104.14) (end 156.08 102.83) (width 0.25) (layer "F.Cu") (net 21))
 (segment (start 154.86 96.95) (end 154.43 96.52) (width 0.25) (layer "F.Cu") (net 21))
 (segment (start 157.48 104.14) (end 157.39 104.14) (width 0.25) (layer "F.Cu") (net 21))
 (segment (start 155.9 119.38) (end 157.48 119.38) (width 1) (layer "F.Cu") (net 27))
 (segment (start 149.2 104.14) (end 148.24 105.1) (width 1) (layer "F.Cu") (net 27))
 (segment (start 148.18 108.262426) (end 148.18 110.986036) (width 1) (layer "F.Cu") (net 27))
 (segment (start 148.24 108.117573) (end 148.24 105.1) (width 1) (layer "F.Cu") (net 27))
 (segment (start 153.202771 118.262771) (end 149.773792 114.833792) (width 1) (layer "F.Cu") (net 27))
 (segment (start 152.49 104.14) (end 149.2 104.14) (width 1) (layer "F.Cu") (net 27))
 (arc (start 148.18 110.986036) (mid 148.594213 113.068426) (end 149.773792 114.833792) (width 1) (layer "F.Cu") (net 27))
 (arc (start 148.24 108.117573) (mid 148.232203 108.15677) (end 148.21 108.19) (width 1) (layer "F.Cu") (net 27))
 (arc (start 153.202771 118.262771) (mid 154.44027 119.089641) (end 155.9 119.38) (width 1) (layer "F.Cu") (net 27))
 (arc (start 148.21 108.19) (mid 148.187796 108.223229) (end 148.18 108.262426) (width 0.25) (layer "F.Cu") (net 27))
 (segment (start 156.76 109.22) (end 157.48 109.22) (width 0.25) (layer "F.Cu") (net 23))
 (segment (start 155.131802 105.031802) (end 156.12 106.02) (width 0.25) (layer "F.Cu") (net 23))
 (segment (start 156.12 108.127451) (end 156.12 106.02) (width 0.25) (layer "F.Cu") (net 23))
 (segment (start 153.93 99.08) (end 153.93 100.218198) (width 0.25) (layer "F.Cu") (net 23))
 (segment (start 153.91 99.06) (end 153.93 99.08) (width 0.25) (layer "F.Cu") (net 23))
 (segment (start 153.93 100.218198) (end 155.131802 101.42) (width 0.25) (layer "F.Cu") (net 23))
 (segment (start 152.49 99.06) (end 153.91 99.06) (width 0.25) (layer "F.Cu") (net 23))
 (segment (start 156.44 108.9) (end 156.76 109.22) (width 0.25) (layer "F.Cu") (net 23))
 (segment (start 155.131802 101.42) (end 155.131802 105.031802) (width 0.25) (layer "F.Cu") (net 23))
 (arc (start 156.12 108.127451) (mid 156.203165 108.545551) (end 156.44 108.9) (width 0.25) (layer "F.Cu") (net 23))
 (segment (start 155.581802 104.781802) (end 157.48 106.68) (width 0.25) (layer "F.Cu") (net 22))
 (segment (start 152.49 97.79) (end 154.08 97.79) (width 0.25) (layer "F.Cu") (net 22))
 (segment (start 155.581802 101.178198) (end 155.581802 104.781802) (width 0.25) (layer "F.Cu") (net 22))
 (segment (start 154.41 98.12) (end 154.41 100.006396) (width 0.25) (layer "F.Cu") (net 22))
 (segment (start 154.08 97.79) (end 154.41 98.12) (width 0.25) (layer "F.Cu") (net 22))
 (segment (start 154.41 100.006396) (end 155.581802 101.178198) (width 0.25) (layer "F.Cu") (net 22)))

